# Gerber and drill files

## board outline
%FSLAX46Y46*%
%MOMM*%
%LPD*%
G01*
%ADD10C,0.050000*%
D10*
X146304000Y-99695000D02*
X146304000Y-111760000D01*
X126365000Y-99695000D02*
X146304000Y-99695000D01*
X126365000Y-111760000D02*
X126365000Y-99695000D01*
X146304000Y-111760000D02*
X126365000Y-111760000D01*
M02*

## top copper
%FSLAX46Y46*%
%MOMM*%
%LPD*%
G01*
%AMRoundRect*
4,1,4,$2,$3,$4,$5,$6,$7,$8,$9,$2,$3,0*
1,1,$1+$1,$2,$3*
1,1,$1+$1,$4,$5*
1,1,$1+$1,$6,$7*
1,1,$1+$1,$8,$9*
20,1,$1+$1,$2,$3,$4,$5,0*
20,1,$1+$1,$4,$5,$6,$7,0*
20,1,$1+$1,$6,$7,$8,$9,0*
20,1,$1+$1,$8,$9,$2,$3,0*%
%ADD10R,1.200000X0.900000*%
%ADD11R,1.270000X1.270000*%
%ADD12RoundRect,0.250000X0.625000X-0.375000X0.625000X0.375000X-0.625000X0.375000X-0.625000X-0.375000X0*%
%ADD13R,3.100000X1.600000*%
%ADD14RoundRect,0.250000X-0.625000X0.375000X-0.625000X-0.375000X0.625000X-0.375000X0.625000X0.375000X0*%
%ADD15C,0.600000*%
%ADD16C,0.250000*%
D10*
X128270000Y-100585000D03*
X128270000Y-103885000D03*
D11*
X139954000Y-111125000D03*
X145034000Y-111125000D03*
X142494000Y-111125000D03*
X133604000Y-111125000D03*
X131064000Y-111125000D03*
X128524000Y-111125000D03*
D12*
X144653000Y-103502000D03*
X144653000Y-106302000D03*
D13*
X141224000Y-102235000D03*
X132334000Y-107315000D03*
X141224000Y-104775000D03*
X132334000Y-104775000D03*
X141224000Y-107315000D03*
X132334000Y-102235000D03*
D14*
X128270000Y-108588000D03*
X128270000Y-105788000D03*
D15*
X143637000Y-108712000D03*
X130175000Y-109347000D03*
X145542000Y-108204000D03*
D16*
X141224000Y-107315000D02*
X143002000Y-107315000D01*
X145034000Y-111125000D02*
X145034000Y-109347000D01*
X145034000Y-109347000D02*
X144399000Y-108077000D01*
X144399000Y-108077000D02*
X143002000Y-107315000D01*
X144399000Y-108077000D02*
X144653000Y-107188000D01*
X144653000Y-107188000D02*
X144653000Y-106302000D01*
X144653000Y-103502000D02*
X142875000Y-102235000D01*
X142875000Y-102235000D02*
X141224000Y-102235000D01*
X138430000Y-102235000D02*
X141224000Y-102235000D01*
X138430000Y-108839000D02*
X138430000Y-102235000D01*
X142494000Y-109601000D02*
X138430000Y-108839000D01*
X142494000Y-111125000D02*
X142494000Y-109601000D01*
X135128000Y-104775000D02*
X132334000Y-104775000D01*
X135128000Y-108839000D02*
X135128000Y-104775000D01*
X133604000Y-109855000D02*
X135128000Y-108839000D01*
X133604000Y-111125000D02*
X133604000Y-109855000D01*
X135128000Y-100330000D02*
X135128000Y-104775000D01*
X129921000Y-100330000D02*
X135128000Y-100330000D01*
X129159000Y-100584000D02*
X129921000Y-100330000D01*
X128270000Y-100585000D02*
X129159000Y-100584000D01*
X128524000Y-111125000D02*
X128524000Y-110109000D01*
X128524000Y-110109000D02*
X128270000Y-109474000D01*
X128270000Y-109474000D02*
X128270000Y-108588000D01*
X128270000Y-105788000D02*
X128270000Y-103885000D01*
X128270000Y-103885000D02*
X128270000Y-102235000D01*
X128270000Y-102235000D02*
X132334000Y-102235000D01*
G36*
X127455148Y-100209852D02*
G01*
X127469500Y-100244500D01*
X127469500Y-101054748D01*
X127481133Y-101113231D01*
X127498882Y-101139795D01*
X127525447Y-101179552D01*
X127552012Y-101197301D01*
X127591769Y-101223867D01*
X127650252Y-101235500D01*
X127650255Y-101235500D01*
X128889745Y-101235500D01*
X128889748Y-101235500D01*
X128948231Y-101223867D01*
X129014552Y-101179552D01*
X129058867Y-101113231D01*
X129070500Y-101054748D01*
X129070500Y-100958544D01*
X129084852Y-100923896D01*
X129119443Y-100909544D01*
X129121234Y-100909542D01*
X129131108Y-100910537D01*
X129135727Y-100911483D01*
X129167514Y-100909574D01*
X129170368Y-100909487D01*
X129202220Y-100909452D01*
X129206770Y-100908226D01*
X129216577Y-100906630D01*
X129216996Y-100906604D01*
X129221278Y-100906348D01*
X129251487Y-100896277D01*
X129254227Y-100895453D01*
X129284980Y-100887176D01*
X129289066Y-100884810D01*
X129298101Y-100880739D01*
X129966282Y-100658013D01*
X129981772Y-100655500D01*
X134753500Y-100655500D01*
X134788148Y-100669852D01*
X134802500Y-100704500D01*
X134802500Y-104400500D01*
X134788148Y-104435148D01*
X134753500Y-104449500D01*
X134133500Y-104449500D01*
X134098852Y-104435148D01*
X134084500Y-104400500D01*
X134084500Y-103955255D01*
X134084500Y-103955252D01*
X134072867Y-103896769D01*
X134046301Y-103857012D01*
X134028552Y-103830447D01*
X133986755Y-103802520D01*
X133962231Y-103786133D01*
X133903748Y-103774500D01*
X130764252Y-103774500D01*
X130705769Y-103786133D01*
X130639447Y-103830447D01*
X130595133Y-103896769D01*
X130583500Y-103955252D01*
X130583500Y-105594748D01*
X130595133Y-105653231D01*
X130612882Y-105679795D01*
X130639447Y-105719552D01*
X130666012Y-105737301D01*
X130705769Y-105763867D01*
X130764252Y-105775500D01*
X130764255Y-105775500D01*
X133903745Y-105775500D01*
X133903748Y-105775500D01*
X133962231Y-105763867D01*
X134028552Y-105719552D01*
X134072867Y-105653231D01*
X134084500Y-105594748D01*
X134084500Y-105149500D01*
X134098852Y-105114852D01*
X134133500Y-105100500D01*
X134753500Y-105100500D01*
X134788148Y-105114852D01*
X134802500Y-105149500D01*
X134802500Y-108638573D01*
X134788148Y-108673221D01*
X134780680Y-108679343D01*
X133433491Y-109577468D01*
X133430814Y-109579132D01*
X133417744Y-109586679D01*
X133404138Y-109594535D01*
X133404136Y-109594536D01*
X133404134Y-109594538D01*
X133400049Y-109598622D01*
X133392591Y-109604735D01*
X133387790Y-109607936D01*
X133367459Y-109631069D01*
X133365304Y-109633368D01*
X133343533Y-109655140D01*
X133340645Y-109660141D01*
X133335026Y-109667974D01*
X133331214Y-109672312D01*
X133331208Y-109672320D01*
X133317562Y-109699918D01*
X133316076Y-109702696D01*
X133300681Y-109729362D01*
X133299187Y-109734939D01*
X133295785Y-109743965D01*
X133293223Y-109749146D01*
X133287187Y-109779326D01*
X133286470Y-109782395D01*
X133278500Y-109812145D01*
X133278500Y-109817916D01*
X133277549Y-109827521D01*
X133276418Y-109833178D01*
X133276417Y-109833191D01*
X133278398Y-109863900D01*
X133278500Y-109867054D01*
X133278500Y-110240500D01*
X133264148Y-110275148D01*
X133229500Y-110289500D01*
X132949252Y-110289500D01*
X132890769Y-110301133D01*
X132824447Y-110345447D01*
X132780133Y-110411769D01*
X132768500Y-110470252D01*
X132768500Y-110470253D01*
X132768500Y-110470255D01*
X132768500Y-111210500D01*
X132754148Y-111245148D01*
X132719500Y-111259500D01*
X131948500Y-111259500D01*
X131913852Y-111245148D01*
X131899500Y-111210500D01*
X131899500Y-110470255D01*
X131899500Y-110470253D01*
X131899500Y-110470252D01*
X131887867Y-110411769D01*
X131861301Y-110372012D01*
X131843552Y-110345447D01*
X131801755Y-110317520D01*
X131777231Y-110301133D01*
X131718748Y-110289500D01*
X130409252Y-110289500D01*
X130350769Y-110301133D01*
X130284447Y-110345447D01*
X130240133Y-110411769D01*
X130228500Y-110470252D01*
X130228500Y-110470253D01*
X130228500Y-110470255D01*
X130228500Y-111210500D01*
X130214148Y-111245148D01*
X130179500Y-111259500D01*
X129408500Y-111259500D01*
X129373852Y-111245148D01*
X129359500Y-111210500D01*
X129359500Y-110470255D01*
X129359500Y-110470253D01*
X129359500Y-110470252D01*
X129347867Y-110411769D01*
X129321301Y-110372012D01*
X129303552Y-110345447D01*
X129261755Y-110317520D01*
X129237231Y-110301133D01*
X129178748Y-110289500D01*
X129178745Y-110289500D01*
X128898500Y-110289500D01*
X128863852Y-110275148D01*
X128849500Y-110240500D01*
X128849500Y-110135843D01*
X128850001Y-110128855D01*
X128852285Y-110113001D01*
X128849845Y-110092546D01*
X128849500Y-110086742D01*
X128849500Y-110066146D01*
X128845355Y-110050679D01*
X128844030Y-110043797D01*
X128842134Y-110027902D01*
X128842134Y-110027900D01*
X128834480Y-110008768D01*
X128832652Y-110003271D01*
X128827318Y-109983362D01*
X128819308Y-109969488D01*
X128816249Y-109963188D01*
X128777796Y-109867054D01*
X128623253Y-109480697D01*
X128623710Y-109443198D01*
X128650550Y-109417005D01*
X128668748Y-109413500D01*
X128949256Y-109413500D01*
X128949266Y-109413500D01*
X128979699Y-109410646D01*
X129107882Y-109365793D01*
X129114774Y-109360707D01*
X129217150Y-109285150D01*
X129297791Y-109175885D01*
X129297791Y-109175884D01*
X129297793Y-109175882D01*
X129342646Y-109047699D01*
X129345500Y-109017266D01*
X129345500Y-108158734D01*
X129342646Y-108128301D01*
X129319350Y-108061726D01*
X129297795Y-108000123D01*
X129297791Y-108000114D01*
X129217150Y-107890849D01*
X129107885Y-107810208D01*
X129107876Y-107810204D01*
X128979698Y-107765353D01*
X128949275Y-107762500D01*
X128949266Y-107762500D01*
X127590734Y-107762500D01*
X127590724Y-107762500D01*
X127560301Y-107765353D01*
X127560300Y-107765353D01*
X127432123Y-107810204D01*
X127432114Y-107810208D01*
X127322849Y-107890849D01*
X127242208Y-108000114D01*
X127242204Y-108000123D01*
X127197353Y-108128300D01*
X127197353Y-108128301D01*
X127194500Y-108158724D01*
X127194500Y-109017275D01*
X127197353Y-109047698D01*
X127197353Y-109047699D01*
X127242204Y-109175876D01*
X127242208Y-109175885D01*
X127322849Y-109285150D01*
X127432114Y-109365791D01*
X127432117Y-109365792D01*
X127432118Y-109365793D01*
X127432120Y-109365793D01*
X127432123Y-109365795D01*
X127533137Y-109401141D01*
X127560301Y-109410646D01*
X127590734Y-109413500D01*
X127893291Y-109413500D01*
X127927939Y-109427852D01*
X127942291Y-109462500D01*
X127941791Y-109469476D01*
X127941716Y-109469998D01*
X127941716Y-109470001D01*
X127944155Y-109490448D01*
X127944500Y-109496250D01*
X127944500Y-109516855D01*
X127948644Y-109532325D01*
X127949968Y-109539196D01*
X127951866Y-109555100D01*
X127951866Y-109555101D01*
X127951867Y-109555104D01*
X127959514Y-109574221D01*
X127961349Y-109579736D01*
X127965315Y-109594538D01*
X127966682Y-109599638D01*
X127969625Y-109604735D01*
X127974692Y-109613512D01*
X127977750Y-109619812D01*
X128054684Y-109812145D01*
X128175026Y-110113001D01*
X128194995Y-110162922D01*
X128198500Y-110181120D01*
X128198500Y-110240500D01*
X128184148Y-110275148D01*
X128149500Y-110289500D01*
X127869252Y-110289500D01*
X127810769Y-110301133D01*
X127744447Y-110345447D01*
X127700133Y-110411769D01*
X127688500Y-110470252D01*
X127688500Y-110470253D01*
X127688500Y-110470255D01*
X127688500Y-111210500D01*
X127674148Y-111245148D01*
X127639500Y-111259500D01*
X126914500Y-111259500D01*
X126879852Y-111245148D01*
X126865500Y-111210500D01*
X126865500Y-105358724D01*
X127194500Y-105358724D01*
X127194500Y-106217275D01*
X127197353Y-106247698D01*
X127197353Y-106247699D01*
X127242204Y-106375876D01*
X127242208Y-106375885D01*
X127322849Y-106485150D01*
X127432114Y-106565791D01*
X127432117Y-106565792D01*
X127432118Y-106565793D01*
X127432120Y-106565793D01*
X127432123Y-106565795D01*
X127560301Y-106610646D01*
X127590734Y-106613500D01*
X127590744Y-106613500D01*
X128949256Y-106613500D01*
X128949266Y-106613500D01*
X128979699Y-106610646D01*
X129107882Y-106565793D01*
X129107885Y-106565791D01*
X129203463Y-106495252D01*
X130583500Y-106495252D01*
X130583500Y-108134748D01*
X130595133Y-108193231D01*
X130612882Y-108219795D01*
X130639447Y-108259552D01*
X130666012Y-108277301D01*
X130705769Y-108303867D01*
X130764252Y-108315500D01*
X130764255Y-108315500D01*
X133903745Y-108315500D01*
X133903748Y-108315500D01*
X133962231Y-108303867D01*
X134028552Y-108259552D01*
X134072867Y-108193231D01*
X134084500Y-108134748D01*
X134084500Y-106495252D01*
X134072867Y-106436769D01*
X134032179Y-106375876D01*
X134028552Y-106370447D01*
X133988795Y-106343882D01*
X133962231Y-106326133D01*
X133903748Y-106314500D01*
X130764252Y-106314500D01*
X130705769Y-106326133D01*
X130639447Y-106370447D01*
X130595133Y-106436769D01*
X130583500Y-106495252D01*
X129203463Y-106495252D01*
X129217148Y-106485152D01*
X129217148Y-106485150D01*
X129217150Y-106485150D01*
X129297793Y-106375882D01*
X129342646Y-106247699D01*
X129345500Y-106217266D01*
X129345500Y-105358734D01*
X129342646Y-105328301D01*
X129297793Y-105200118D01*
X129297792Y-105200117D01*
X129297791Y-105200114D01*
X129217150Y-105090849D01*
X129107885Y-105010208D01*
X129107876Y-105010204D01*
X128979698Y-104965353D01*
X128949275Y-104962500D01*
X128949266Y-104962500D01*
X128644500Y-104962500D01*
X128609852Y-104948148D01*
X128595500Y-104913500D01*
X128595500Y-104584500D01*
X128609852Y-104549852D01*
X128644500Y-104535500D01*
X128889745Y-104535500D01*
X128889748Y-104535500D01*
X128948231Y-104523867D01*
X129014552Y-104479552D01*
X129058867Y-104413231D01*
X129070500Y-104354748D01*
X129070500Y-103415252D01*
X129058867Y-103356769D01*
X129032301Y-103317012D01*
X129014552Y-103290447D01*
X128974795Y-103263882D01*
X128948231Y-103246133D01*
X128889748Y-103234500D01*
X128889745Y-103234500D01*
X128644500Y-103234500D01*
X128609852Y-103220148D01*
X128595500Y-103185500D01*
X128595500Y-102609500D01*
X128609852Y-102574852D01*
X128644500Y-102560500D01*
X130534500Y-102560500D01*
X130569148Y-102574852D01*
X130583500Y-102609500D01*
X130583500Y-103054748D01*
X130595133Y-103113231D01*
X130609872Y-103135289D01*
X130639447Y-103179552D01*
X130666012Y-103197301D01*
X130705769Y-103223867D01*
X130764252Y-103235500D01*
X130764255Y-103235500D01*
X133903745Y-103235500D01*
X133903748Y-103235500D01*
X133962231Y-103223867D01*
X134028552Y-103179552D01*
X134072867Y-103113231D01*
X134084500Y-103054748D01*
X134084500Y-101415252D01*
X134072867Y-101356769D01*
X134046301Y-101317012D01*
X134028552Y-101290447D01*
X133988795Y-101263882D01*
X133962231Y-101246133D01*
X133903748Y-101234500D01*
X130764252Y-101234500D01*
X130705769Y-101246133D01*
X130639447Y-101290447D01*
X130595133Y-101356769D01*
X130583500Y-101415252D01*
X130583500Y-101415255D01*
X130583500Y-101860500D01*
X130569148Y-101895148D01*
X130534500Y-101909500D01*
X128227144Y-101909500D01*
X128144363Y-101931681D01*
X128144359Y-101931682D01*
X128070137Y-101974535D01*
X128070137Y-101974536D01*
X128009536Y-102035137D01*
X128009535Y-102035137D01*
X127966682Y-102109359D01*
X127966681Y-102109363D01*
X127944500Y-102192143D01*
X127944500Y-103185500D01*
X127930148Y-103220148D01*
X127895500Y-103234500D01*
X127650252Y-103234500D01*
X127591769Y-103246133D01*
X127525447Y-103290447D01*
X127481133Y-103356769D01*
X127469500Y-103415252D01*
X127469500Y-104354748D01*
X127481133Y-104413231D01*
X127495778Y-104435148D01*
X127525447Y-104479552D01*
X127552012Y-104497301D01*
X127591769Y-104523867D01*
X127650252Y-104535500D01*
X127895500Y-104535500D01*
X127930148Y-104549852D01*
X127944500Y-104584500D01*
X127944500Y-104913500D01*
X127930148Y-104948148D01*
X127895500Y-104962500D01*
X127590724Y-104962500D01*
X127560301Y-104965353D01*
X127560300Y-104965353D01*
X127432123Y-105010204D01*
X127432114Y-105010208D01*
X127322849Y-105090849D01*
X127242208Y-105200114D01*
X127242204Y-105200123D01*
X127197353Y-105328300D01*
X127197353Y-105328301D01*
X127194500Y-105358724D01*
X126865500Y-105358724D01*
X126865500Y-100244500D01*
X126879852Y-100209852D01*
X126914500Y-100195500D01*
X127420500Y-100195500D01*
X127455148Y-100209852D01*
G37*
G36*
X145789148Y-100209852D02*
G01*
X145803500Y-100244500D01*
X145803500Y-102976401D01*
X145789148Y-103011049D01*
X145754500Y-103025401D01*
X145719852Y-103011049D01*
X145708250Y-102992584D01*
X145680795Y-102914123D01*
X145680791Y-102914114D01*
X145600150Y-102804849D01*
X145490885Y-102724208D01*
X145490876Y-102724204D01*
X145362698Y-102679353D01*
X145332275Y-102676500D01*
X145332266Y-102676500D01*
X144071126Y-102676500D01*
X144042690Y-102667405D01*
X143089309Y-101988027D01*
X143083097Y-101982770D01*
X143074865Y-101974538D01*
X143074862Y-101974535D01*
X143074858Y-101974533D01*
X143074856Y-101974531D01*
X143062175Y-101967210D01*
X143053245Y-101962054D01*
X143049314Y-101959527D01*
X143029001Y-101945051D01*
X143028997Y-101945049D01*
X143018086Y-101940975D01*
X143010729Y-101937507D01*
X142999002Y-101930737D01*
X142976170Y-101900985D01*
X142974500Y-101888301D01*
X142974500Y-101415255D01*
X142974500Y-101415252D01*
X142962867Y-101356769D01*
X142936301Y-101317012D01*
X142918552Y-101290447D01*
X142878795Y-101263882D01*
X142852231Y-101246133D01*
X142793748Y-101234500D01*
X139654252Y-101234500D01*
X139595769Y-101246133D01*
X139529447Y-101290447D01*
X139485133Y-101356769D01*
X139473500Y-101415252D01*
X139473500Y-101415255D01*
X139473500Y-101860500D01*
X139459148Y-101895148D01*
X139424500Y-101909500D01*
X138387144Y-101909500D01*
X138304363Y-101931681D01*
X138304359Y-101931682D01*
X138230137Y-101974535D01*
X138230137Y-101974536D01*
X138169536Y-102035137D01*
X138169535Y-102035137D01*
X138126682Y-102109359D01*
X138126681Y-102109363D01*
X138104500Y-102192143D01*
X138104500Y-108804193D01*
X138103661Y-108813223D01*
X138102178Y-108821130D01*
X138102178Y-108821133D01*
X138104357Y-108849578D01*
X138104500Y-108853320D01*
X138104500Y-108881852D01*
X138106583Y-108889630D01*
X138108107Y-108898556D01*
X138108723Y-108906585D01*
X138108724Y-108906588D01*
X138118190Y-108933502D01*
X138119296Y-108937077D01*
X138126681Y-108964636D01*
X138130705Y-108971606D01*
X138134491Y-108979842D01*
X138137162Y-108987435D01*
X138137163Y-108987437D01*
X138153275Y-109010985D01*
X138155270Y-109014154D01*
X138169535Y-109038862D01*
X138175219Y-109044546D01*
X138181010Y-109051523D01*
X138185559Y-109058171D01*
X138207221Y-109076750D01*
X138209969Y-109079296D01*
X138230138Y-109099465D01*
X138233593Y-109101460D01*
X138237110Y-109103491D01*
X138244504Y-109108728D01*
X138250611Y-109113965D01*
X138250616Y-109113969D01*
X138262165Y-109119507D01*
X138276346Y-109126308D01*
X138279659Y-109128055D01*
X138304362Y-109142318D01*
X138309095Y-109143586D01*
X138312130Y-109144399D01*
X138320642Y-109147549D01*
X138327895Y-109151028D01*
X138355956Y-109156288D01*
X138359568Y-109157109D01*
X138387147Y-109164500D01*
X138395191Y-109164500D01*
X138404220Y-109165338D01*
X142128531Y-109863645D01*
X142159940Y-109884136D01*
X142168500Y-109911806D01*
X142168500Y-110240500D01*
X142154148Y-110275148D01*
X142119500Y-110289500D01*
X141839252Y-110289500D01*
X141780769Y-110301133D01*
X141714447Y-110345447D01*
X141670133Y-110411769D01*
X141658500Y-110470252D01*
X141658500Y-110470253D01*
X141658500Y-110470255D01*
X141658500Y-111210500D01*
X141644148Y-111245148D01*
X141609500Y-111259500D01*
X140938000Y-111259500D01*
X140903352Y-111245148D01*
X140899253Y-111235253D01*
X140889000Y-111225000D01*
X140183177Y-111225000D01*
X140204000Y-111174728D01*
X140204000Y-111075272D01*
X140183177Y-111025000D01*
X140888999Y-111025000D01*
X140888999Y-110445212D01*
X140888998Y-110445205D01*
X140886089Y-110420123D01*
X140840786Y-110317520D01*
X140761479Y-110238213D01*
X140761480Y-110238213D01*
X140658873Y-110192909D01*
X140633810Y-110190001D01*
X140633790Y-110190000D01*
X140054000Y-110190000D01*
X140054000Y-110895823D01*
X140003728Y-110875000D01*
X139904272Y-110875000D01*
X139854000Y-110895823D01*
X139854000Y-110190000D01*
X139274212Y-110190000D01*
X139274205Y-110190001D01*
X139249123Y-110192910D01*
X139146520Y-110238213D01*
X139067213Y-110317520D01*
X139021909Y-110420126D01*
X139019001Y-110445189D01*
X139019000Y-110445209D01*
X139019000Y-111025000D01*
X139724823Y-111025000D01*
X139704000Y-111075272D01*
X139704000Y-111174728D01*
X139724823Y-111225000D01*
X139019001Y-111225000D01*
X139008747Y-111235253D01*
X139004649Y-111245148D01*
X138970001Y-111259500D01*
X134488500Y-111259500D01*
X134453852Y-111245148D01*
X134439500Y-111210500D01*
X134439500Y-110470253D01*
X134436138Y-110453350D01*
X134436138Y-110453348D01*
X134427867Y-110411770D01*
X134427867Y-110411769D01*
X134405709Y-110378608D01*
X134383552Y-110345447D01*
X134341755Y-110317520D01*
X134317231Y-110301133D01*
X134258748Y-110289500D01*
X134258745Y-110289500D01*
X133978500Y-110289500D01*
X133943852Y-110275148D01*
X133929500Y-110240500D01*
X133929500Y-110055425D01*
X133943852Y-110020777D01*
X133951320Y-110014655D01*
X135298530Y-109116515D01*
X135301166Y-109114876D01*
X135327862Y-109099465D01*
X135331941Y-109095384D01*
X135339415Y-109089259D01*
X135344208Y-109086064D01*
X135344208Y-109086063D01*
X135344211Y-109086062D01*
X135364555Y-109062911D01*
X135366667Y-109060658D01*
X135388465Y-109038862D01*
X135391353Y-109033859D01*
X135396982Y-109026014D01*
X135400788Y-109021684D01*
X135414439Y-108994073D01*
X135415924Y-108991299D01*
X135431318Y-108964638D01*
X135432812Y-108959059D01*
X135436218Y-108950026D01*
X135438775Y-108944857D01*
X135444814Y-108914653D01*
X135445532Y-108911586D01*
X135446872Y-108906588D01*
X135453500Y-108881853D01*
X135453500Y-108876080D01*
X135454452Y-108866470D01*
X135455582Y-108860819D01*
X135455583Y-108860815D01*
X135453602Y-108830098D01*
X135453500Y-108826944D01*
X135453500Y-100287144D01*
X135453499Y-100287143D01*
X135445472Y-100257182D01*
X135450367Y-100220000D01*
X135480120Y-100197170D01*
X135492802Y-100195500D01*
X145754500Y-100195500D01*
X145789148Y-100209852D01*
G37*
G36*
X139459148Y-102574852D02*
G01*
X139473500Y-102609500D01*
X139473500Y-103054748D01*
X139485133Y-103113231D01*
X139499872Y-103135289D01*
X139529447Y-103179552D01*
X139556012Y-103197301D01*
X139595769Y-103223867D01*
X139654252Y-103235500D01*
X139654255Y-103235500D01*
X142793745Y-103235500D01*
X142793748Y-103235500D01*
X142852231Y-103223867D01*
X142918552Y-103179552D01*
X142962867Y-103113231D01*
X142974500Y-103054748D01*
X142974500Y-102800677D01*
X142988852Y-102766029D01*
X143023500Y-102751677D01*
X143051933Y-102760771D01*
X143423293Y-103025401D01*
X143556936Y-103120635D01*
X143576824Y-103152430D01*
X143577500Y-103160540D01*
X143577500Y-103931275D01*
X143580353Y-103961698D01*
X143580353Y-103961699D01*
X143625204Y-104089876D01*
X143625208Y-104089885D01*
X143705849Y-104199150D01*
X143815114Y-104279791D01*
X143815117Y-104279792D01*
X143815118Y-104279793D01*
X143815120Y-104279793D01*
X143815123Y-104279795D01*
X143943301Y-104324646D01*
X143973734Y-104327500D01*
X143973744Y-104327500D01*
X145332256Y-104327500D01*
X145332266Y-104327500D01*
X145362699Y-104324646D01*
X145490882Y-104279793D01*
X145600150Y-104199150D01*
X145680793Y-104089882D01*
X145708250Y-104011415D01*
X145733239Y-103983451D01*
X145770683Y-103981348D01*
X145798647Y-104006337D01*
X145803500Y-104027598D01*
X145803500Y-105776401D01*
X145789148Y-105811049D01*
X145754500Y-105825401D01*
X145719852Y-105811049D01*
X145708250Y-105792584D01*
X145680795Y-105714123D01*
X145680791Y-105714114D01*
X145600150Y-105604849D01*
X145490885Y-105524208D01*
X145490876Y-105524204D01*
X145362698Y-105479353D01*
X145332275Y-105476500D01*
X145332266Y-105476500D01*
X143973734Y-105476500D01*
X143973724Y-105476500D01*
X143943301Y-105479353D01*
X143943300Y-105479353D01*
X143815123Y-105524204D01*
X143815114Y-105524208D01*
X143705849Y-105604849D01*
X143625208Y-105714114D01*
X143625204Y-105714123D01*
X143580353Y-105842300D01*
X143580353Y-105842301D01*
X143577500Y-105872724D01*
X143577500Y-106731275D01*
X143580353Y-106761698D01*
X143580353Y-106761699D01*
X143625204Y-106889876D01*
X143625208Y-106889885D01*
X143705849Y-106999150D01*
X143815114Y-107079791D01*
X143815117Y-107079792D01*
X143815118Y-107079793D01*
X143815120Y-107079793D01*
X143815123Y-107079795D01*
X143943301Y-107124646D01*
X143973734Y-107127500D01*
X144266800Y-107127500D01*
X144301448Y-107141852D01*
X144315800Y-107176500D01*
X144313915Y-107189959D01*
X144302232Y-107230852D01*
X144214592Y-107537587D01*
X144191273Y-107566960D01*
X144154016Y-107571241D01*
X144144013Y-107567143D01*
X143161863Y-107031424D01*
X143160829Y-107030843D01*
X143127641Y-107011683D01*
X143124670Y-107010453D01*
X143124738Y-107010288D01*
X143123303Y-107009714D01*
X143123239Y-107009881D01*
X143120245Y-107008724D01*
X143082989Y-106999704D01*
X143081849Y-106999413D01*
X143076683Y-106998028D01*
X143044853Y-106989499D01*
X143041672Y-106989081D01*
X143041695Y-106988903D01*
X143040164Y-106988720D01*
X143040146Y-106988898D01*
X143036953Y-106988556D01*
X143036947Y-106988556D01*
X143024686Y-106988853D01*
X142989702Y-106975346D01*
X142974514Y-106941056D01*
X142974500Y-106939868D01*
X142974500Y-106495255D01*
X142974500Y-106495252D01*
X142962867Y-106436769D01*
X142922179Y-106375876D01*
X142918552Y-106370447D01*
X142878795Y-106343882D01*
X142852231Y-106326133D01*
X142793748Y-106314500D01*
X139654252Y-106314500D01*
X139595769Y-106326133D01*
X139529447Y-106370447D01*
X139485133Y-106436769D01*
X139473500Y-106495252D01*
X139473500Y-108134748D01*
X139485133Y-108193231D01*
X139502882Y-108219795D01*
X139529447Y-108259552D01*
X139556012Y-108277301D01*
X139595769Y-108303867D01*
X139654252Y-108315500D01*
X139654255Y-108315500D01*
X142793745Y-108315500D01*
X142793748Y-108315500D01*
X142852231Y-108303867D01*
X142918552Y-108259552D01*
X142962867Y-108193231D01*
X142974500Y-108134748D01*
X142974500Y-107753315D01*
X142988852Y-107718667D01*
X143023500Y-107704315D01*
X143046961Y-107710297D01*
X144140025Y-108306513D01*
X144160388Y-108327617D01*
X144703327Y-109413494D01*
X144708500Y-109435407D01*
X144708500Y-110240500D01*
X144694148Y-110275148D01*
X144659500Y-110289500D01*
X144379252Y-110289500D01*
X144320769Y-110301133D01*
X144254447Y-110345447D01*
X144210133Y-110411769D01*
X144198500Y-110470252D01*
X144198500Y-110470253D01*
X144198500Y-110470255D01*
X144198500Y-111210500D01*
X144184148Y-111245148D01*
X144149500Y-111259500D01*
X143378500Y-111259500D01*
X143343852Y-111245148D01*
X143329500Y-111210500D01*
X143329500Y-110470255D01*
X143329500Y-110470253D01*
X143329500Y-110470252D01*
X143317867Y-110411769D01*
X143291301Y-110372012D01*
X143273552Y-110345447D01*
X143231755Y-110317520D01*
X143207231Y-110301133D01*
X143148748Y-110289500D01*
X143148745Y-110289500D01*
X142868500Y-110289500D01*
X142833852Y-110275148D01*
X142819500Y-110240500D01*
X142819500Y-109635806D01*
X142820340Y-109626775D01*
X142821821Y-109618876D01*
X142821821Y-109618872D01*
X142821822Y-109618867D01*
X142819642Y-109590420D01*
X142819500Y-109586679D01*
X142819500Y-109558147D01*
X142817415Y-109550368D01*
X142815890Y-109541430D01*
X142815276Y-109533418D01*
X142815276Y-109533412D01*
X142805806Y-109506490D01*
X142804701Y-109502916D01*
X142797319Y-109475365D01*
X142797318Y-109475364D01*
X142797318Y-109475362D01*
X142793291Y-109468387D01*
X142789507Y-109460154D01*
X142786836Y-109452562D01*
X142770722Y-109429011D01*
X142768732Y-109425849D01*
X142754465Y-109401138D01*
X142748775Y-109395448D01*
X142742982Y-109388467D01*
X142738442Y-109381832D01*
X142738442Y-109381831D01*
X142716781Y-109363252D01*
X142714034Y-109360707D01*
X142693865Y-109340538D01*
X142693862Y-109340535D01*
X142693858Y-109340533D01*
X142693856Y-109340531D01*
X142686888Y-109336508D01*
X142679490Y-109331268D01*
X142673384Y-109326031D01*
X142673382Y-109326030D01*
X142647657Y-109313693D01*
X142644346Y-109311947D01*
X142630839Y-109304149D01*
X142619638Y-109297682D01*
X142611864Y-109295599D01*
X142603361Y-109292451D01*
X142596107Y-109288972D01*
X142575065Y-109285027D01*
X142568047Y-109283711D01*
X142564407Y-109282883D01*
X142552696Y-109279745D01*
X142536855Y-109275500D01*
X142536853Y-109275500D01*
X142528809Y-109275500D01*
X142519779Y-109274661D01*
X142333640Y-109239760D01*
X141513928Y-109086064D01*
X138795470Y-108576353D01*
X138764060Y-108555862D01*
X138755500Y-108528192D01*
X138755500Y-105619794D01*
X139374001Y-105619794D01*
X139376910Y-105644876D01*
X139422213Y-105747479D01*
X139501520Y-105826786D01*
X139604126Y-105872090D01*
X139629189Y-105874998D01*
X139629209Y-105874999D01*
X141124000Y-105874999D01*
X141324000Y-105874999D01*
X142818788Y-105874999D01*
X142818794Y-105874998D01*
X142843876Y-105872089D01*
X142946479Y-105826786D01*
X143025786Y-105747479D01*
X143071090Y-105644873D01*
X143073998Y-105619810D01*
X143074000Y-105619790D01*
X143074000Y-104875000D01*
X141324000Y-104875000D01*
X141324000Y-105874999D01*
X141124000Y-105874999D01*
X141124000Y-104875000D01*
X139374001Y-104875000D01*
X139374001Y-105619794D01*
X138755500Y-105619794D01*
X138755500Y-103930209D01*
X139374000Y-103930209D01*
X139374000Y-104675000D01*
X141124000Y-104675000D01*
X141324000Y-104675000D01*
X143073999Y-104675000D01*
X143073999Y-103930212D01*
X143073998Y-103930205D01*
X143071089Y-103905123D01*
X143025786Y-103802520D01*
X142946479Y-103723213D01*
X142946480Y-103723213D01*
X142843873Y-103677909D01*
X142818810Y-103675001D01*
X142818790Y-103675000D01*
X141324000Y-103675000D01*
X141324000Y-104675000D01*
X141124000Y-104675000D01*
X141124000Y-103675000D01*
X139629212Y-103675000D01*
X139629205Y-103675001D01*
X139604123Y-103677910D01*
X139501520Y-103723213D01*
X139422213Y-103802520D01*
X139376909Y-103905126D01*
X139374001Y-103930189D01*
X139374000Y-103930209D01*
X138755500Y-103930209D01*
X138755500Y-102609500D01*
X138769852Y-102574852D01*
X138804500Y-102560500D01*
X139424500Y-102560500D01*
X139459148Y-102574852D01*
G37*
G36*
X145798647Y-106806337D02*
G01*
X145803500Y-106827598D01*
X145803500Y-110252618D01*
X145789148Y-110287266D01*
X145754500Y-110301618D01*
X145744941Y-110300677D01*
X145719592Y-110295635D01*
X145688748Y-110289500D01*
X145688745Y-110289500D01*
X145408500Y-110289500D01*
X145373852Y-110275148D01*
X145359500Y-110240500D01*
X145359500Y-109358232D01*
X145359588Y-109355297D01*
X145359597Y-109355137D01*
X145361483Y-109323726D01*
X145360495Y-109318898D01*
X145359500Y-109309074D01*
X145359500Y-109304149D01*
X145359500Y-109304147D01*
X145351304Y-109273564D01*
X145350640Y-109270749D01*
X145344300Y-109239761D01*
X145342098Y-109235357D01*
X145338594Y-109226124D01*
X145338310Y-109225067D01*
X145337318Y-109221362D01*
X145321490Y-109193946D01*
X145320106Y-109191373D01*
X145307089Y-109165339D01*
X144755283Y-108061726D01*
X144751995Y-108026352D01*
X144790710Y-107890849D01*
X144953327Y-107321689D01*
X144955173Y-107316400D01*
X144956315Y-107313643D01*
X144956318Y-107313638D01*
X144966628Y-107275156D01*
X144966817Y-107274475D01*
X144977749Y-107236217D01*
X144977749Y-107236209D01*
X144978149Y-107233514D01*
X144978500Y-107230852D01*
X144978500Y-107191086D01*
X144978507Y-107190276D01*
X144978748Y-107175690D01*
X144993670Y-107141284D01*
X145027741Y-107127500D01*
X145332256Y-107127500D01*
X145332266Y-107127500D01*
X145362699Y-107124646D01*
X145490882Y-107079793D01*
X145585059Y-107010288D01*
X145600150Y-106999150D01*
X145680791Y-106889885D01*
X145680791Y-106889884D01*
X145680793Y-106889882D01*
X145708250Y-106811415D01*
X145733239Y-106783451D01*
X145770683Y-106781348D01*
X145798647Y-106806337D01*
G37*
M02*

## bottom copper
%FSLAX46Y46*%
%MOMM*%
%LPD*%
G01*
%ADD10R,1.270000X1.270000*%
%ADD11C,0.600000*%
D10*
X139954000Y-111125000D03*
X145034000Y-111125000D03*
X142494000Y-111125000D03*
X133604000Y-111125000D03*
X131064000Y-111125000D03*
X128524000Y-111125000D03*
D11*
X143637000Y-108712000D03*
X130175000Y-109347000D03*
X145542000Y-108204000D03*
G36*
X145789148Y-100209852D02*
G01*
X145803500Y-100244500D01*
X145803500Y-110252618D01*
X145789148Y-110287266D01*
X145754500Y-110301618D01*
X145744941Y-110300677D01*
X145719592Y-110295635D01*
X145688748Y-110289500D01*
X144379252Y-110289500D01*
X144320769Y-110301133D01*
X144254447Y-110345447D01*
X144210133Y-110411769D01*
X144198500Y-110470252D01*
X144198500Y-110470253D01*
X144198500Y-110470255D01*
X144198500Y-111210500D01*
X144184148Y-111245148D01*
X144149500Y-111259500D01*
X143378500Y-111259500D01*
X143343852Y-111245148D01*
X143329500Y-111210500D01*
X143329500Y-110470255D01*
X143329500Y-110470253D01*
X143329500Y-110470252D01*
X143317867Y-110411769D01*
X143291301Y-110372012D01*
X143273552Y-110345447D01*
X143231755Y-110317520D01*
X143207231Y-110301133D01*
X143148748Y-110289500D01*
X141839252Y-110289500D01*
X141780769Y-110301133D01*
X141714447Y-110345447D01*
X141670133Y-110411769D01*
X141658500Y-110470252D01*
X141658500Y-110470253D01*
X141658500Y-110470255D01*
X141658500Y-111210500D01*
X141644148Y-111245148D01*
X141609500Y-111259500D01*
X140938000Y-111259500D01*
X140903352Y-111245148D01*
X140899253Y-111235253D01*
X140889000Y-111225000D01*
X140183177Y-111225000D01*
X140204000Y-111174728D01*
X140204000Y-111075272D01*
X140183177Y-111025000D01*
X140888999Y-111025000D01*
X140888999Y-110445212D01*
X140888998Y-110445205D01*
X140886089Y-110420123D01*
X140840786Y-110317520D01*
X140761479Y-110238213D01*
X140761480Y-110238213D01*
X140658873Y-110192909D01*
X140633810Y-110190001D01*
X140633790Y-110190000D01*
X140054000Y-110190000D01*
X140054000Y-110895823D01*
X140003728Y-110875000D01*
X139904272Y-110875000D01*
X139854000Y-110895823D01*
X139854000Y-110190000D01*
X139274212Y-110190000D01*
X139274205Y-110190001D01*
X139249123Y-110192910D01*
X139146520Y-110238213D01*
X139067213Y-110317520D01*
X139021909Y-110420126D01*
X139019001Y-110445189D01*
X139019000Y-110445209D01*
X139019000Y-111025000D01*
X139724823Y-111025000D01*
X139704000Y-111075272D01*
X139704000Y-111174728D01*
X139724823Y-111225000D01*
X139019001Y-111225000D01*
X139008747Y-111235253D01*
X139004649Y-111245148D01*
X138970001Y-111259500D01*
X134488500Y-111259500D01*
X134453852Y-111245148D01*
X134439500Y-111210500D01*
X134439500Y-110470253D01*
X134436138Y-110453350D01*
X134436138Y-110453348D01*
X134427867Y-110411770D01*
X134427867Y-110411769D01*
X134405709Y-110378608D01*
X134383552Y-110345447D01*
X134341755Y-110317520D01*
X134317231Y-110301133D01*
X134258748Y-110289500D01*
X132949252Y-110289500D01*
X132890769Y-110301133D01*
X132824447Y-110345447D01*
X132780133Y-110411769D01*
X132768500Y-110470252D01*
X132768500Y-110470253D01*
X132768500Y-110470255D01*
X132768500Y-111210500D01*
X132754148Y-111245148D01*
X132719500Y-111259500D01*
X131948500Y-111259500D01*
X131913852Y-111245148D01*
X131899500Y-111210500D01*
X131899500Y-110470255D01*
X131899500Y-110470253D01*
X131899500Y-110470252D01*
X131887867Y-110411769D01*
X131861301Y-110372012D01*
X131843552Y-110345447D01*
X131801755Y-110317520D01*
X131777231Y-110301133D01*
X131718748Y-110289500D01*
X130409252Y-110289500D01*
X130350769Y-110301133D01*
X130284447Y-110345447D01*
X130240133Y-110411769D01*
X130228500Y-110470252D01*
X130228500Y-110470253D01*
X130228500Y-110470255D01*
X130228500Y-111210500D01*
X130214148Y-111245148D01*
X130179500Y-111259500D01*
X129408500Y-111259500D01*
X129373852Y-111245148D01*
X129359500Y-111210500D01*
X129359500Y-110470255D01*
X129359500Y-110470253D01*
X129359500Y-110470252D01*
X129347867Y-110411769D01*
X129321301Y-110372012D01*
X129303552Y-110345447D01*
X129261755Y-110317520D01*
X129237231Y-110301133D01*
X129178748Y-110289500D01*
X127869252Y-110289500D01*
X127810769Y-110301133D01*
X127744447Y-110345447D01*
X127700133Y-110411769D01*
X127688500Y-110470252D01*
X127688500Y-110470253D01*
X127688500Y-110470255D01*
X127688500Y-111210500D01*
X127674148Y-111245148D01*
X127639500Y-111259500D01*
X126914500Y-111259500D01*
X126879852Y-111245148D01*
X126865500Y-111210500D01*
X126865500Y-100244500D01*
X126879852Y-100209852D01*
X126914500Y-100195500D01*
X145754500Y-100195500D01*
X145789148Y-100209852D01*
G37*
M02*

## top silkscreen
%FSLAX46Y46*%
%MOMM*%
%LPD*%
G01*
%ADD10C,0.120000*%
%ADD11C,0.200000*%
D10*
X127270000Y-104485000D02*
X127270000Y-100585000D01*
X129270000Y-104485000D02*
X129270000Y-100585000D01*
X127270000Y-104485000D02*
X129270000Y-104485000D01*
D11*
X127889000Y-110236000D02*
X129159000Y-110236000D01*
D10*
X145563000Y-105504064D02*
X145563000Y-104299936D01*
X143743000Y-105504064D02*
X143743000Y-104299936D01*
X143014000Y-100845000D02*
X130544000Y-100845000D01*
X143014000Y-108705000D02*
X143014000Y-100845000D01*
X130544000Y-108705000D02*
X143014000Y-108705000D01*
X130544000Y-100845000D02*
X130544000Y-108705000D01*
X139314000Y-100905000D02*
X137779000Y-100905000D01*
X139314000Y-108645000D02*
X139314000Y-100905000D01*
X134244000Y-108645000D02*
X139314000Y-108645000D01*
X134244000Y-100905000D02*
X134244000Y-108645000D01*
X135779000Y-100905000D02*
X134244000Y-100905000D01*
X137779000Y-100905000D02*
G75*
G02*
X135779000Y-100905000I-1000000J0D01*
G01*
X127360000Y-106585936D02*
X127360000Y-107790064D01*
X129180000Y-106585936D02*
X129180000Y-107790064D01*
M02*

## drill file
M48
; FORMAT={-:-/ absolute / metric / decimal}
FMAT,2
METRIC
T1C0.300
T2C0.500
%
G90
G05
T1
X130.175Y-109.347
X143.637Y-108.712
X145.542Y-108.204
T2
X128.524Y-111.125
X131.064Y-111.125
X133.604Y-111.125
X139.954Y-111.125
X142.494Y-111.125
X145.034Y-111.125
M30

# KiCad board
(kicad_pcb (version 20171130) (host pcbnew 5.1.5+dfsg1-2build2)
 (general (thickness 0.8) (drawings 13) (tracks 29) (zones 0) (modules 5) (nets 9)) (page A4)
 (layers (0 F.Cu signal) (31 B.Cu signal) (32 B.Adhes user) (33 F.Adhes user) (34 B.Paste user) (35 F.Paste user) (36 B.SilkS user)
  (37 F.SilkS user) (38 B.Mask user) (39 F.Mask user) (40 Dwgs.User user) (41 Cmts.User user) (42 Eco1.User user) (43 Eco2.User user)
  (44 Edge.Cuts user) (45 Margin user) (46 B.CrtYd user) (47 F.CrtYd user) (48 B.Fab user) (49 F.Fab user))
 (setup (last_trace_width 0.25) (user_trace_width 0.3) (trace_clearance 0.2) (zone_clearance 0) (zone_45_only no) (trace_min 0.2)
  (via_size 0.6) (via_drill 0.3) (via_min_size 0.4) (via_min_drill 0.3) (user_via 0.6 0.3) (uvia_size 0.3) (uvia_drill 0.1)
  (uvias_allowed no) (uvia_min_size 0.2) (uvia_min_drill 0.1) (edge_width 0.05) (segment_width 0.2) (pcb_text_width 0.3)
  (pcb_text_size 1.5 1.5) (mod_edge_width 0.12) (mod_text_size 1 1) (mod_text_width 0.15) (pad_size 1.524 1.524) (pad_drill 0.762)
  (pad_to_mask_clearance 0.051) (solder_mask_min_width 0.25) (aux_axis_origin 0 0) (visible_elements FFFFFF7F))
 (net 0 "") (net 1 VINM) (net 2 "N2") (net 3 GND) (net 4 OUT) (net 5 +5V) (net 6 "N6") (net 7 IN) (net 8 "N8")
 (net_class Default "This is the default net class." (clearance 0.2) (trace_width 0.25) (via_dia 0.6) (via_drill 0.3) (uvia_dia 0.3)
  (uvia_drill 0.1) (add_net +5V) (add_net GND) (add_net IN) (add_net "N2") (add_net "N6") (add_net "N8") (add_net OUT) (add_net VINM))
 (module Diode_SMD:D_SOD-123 (layer F.Cu) (at 128.27 102.235 90)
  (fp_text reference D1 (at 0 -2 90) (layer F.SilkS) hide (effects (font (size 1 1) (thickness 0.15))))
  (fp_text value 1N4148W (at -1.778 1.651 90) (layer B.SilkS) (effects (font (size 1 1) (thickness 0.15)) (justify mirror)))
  (fp_line (start -2.25 -1) (end 1.65 -1) (layer F.SilkS) (width 0.12))
  (fp_line (start -2.25 1) (end 1.65 1) (layer F.SilkS) (width 0.12))
  (fp_line (start -2.25 -1) (end -2.25 1) (layer F.SilkS) (width 0.12))
  (pad 2 smd rect (at 1.65 0 90) (size 0.9 1.2) (layers F.Cu F.Paste F.Mask) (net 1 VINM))
  (pad 1 smd rect (at -1.65 0 90) (size 0.9 1.2) (layers F.Cu F.Paste F.Mask) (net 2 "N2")))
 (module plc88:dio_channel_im (layer F.Cu) (at 135.509 108.585)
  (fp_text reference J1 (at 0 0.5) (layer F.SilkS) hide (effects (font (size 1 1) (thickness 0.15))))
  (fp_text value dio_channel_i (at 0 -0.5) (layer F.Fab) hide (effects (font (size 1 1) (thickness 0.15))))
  (fp_line (start -7.62 1.651) (end -6.35 1.651) (layer F.SilkS) (width 0.2))
  (pad 4 thru_hole rect (at 4.445 2.54) (size 1.27 1.27) (drill 0.5) (layers *.Cu *.Mask) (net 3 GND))
  (pad 6 thru_hole rect (at 9.525 2.54) (size 1.27 1.27) (drill 0.5) (layers *.Cu *.Mask) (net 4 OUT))
  (pad 5 thru_hole rect (at 6.985 2.54) (size 1.27 1.27) (drill 0.5) (layers *.Cu *.Mask) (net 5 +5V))
  (pad 3 thru_hole rect (at -1.905 2.54) (size 1.27 1.27) (drill 0.5) (layers *.Cu *.Mask) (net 1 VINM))
  (pad 2 thru_hole rect (at -4.445 2.54) (size 1.27 1.27) (drill 0.5) (layers *.Cu *.Mask) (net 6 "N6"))
  (pad 1 thru_hole rect (at -6.985 2.54) (size 1.27 1.27) (drill 0.5) (layers *.Cu *.Mask) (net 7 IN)))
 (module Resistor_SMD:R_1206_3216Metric (layer F.Cu) (at 144.653 104.902 90)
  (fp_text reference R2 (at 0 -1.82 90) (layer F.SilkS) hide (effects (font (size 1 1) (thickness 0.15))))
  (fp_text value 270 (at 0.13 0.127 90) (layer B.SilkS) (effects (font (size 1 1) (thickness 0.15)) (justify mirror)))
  (fp_line (start -0.602064 0.91) (end 0.602064 0.91) (layer F.SilkS) (width 0.12))
  (fp_line (start -0.602064 -0.91) (end 0.602064 -0.91) (layer F.SilkS) (width 0.12))
  (pad 2 smd roundrect (at 1.4 0 90) (size 1.25 1.75) (layers F.Cu F.Paste F.Mask) (roundrect_rratio 0.2) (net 5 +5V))
  (pad 1 smd roundrect (at -1.4 0 90) (size 1.25 1.75) (layers F.Cu F.Paste F.Mask) (roundrect_rratio 0.2) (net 4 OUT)))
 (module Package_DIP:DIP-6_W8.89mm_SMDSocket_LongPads (layer F.Cu) (at 136.779 104.775)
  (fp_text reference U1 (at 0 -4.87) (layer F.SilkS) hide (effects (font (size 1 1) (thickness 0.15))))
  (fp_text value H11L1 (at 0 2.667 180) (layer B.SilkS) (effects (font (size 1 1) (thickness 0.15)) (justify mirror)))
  (fp_line (start 6.235 -3.93) (end -6.235 -3.93) (layer F.SilkS) (width 0.12))
  (fp_line (start 6.235 3.93) (end 6.235 -3.93) (layer F.SilkS) (width 0.12))
  (fp_line (start -6.235 3.93) (end 6.235 3.93) (layer F.SilkS) (width 0.12))
  (fp_line (start -6.235 -3.93) (end -6.235 3.93) (layer F.SilkS) (width 0.12))
  (fp_line (start 2.535 -3.87) (end 1 -3.87) (layer F.SilkS) (width 0.12))
  (fp_line (start 2.535 3.87) (end 2.535 -3.87) (layer F.SilkS) (width 0.12))
  (fp_line (start -2.535 3.87) (end 2.535 3.87) (layer F.SilkS) (width 0.12))
  (fp_line (start -2.535 -3.87) (end -2.535 3.87) (layer F.SilkS) (width 0.12))
  (fp_line (start -1 -3.87) (end -2.535 -3.87) (layer F.SilkS) (width 0.12))
  (fp_arc (start 0 -3.87) (end -1 -3.87) (angle -180) (layer F.SilkS) (width 0.12))
  (pad 6 smd rect (at 4.445 -2.54) (size 3.1 1.6) (layers F.Cu F.Paste F.Mask) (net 5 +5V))
  (pad 3 smd rect (at -4.445 2.54) (size 3.1 1.6) (layers F.Cu F.Paste F.Mask) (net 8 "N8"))
  (pad 5 smd rect (at 4.445 0) (size 3.1 1.6) (layers F.Cu F.Paste F.Mask) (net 3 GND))
  (pad 2 smd rect (at -4.445 0) (size 3.1 1.6) (layers F.Cu F.Paste F.Mask) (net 1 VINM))
  (pad 4 smd rect (at 4.445 2.54) (size 3.1 1.6) (layers F.Cu F.Paste F.Mask) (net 4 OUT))
  (pad 1 smd rect (at -4.445 -2.54) (size 3.1 1.6) (layers F.Cu F.Paste F.Mask) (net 2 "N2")))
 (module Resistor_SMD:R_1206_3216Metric (layer F.Cu) (at 128.27 107.188 270)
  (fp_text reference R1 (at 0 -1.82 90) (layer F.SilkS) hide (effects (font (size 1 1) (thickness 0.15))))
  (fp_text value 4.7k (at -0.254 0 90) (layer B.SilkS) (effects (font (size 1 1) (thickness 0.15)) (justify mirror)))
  (fp_line (start -0.602064 0.91) (end 0.602064 0.91) (layer F.SilkS) (width 0.12))
  (fp_line (start -0.602064 -0.91) (end 0.602064 -0.91) (layer F.SilkS) (width 0.12))
  (pad 2 smd roundrect (at 1.4 0 270) (size 1.25 1.75) (layers F.Cu F.Paste F.Mask) (roundrect_rratio 0.2) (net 7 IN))
  (pad 1 smd roundrect (at -1.4 0 270) (size 1.25 1.75) (layers F.Cu F.Paste F.Mask) (roundrect_rratio 0.2) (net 2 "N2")))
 (gr_line (start 146.304 99.695) (end 146.304 111.76) (layer Edge.Cuts) (width 0.05))
 (gr_line (start 126.365 99.695) (end 146.304 99.695) (layer Edge.Cuts) (width 0.05))
 (gr_line (start 126.365 111.76) (end 126.365 99.695) (layer Edge.Cuts) (width 0.05))
 (gr_line (start 146.304 111.76) (end 126.365 111.76) (layer Edge.Cuts) (width 0.05))
 (segment (start 141.224 107.315) (end 143.002 107.315) (width 0.25) (layer F.Cu) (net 4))
 (segment (start 145.034 111.125) (end 145.034 109.347) (width 0.25) (layer F.Cu) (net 4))
 (segment (start 145.034 109.347) (end 144.399 108.077) (width 0.25) (layer F.Cu) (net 4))
 (segment (start 144.399 108.077) (end 143.002 107.315) (width 0.25) (layer F.Cu) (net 4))
 (segment (start 144.399 108.077) (end 144.653 107.188) (width 0.25) (layer F.Cu) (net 4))
 (segment (start 144.653 107.188) (end 144.653 106.302) (width 0.25) (layer F.Cu) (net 4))
 (segment (start 144.653 103.502) (end 142.875 102.235) (width 0.25) (layer F.Cu) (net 5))
 (segment (start 142.875 102.235) (end 141.224 102.235) (width 0.25) (layer F.Cu) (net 5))
 (segment (start 138.43 102.235) (end 141.224 102.235) (width 0.25) (layer F.Cu) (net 5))
 (segment (start 138.43 108.839) (end 138.43 102.235) (width 0.25) (layer F.Cu) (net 5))
 (segment (start 142.494 109.601) (end 138.43 108.839) (width 0.25) (layer F.Cu) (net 5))
 (segment (start 142.494 111.125) (end 142.494 109.601) (width 0.25) (layer F.Cu) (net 5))
 (via (at 143.637 108.712) (size 0.6) (drill 0.3) (layers F.Cu B.Cu) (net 3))
 (via (at 130.175 109.347) (size 0.6) (drill 0.3) (layers F.Cu B.Cu) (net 3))
 (via (at 145.542 108.204) (size 0.6) (drill 0.3) (layers F.Cu B.Cu) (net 3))
 (segment (start 135.128 104.775) (end 132.334 104.775) (width 0.25) (layer F.Cu) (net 1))
 (segment (start 135.128 108.839) (end 135.128 104.775) (width 0.25) (layer F.Cu) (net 1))
 (segment (start 133.604 109.855) (end 135.128 108.839) (width 0.25) (layer F.Cu) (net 1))
 (segment (start 133.604 111.125) (end 133.604 109.855) (width 0.25) (layer F.Cu) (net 1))
 (segment (start 135.128 100.33) (end 135.128 104.775) (width 0.25) (layer F.Cu) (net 1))
 (segment (start 129.921 100.33) (end 135.128 100.33) (width 0.25) (layer F.Cu) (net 1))
 (segment (start 129.159 100.584) (end 129.921 100.33) (width 0.25) (layer F.Cu) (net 1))
 (segment (start 128.27 100.585) (end 129.159 100.584) (width 0.25) (layer F.Cu) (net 1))
 (segment (start 128.524 111.125) (end 128.524 110.109) (width 0.25) (layer F.Cu) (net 7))
 (segment (start 128.524 110.109) (end 128.27 109.474) (width 0.25) (layer F.Cu) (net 7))
 (segment (start 128.27 109.474) (end 128.27 108.588) (width 0.25) (layer F.Cu) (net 7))
 (segment (start 128.27 105.788) (end 128.27 103.885) (width 0.25) (layer F.Cu) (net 2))
 (segment (start 128.27 103.885) (end 128.27 102.235) (width 0.25) (layer F.Cu) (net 2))
 (segment (start 128.27 102.235) (end 132.334 102.235) (width 0.25) (layer F.Cu) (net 2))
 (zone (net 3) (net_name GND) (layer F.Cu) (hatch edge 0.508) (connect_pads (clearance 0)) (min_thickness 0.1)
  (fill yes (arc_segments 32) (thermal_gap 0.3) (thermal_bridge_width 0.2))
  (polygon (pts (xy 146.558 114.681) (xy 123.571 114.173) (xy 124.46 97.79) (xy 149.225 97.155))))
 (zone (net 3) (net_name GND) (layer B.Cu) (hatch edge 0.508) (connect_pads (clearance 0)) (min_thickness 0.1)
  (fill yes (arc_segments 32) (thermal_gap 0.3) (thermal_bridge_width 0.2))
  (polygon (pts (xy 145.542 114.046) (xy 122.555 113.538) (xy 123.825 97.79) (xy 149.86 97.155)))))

